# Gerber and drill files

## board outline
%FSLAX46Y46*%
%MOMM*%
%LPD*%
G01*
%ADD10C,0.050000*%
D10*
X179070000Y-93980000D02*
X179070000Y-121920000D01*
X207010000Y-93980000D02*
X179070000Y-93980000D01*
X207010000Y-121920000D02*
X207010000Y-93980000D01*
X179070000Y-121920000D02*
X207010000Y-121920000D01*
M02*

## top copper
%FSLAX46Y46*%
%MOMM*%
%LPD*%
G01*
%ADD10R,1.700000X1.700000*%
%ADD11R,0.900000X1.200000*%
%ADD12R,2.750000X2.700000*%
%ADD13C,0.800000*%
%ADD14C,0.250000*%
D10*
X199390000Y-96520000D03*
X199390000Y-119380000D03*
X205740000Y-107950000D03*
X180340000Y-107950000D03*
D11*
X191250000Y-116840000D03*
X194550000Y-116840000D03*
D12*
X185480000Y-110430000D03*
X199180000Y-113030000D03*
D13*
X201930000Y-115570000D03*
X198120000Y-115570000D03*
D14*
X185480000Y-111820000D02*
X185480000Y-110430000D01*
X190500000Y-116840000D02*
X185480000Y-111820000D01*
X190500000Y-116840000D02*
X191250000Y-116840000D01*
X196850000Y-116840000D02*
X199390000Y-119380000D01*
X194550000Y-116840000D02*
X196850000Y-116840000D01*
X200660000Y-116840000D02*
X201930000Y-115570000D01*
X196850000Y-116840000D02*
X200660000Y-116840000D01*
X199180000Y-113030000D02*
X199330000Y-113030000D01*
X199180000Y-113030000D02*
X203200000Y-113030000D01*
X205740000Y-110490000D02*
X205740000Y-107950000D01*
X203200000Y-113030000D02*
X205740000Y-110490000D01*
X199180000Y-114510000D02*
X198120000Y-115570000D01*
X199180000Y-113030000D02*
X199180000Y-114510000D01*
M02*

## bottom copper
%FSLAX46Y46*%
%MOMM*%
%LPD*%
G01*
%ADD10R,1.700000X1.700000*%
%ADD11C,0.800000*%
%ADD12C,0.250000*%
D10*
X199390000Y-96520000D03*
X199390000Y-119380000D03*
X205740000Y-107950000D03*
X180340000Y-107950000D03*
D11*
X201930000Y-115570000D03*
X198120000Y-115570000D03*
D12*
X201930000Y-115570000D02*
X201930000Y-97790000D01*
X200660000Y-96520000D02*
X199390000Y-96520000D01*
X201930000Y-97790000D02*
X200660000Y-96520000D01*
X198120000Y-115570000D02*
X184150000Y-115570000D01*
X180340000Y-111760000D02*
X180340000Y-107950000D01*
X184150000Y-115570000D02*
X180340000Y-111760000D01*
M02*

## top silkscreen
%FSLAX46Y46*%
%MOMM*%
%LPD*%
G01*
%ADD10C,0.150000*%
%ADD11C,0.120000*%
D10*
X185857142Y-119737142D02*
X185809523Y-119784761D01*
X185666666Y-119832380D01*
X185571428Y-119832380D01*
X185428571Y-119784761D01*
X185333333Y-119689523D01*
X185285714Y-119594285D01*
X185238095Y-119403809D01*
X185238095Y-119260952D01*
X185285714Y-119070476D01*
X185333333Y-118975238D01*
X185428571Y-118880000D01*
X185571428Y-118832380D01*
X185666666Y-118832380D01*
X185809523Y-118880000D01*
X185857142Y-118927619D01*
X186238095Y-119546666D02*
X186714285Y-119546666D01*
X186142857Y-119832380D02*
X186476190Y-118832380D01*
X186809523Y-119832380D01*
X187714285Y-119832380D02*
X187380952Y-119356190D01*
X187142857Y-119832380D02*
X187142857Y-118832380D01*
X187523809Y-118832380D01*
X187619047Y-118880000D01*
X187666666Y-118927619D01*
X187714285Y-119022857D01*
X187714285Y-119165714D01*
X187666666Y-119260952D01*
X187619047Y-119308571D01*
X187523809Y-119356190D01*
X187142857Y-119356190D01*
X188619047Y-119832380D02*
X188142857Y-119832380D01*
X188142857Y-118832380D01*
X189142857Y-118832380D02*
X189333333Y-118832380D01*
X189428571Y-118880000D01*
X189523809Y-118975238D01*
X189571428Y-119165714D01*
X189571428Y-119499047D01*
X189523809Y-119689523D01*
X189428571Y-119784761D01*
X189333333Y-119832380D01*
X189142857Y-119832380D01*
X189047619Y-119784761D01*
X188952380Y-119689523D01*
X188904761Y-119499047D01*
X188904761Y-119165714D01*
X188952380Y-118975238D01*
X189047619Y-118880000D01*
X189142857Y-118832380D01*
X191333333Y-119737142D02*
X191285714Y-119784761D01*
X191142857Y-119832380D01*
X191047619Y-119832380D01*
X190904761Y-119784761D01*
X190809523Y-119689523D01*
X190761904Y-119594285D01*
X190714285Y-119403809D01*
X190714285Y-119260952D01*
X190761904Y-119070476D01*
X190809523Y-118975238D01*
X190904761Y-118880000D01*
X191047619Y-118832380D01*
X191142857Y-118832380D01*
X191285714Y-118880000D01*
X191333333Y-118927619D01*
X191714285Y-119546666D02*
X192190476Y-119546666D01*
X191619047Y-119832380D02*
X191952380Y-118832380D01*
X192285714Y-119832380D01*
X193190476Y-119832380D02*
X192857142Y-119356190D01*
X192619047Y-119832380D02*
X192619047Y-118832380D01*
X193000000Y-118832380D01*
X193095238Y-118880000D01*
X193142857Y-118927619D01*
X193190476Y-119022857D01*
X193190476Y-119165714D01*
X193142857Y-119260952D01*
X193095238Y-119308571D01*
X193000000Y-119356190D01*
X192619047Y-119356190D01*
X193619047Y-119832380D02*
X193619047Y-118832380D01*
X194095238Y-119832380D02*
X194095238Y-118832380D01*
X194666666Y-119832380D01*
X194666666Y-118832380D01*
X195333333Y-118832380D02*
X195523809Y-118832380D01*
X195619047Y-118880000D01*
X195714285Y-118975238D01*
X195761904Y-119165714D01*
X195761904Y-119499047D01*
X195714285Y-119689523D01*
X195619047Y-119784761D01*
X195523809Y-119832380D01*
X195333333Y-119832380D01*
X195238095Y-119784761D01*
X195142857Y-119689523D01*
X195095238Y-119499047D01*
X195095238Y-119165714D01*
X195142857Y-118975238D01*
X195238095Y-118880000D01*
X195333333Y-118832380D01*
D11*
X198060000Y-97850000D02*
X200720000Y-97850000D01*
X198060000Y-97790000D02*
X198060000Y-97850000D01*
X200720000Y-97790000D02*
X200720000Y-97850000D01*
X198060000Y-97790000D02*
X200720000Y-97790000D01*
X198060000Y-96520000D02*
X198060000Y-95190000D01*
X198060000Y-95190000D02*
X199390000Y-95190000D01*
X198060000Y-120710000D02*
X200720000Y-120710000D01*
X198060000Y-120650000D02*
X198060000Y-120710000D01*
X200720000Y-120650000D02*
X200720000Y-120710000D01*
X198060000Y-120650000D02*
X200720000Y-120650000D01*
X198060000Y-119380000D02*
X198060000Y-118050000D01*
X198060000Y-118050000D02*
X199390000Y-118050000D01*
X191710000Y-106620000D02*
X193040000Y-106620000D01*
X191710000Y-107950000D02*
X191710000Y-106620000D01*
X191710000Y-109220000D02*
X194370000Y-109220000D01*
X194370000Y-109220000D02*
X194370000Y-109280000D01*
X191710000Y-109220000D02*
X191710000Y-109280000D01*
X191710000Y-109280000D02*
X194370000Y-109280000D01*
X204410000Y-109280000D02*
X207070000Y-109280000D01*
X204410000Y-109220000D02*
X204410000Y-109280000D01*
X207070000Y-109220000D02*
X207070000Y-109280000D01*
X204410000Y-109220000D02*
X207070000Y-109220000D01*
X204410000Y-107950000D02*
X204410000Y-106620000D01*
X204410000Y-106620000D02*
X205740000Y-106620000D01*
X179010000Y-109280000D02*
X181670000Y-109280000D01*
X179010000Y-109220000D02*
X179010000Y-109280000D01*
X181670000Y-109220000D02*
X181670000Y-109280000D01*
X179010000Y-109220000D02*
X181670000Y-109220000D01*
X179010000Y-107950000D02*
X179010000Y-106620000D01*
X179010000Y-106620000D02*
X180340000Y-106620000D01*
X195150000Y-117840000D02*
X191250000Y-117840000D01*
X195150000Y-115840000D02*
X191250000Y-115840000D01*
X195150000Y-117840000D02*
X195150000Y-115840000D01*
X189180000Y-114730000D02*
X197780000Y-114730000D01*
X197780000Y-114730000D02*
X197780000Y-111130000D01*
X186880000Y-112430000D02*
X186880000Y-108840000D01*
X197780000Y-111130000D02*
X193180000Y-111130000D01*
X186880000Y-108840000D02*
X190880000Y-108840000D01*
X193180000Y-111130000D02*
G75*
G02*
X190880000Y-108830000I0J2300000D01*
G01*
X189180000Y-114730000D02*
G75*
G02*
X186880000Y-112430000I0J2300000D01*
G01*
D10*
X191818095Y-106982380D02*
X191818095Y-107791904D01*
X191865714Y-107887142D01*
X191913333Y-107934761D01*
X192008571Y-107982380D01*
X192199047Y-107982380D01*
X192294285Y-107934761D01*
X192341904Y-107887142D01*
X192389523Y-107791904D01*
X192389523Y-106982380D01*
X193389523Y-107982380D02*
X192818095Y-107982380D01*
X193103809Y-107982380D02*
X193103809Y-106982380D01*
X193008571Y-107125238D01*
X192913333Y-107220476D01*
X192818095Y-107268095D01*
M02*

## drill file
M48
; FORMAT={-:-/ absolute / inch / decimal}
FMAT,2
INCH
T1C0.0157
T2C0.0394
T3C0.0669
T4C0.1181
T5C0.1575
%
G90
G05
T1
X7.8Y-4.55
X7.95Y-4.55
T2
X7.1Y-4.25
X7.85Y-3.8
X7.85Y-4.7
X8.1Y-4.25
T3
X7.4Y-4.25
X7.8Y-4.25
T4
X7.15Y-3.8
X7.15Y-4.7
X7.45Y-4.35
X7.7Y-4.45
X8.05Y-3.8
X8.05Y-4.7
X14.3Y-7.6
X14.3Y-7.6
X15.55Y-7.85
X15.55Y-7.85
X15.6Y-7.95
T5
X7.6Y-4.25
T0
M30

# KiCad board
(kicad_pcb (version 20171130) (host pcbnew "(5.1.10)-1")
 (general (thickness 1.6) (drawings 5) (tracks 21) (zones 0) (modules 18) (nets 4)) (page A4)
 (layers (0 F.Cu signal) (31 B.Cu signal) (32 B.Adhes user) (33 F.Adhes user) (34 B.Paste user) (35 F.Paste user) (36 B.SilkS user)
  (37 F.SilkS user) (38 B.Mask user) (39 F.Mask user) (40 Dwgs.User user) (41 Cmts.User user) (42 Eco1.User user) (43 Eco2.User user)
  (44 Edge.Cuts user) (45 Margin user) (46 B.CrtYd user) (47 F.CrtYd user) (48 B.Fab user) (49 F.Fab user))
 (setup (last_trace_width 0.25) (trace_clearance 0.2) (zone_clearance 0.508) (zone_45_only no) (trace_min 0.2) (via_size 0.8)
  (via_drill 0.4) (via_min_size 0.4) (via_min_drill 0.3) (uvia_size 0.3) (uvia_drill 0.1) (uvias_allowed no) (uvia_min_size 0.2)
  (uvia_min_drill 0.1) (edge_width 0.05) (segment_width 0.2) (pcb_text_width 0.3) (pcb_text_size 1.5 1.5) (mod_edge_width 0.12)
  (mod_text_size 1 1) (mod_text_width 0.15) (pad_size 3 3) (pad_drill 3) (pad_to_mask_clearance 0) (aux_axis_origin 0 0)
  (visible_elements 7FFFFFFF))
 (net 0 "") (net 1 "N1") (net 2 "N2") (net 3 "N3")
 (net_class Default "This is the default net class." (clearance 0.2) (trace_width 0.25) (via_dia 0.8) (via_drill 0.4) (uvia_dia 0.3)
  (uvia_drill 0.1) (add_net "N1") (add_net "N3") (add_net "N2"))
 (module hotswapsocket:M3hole (layer F.Cu) (at 204.47 96.52)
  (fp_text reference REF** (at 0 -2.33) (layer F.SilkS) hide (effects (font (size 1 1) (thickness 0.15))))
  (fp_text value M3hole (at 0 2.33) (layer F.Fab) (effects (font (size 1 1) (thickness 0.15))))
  (pad "" np_thru_hole circle (at 0 0) (size 3 3) (drill 3) (layers *.Cu *.Mask)))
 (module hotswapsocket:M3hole (layer F.Cu) (at 181.61 119.38)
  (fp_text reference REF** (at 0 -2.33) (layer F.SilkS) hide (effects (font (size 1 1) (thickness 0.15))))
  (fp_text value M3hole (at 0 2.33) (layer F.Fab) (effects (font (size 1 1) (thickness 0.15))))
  (pad "" np_thru_hole circle (at 0 0) (size 3 3) (drill 3) (layers *.Cu *.Mask)))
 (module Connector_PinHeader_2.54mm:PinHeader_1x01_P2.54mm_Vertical (layer F.Cu) (at 204.47 119.38)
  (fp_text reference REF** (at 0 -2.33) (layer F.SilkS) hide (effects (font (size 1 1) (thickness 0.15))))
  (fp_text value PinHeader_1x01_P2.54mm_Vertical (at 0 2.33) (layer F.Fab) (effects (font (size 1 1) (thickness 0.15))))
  (pad "" np_thru_hole circle (at 0 0) (size 3 3) (drill 3) (layers *.Cu *.Mask)))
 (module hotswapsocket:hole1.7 (layer F.Cu) (at 198.12 107.95)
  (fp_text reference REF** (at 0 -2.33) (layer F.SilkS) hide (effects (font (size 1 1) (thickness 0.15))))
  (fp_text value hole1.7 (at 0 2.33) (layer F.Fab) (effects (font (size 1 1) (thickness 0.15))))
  (pad "" np_thru_hole circle (at 0 0) (size 1.7 1.7) (drill 1.7) (layers *.Cu *.Mask)))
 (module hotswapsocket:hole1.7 (layer F.Cu) (at 187.96 107.95)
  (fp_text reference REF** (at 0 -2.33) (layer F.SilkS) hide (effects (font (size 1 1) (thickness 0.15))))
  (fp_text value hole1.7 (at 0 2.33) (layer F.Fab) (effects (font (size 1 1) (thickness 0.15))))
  (pad "" np_thru_hole circle (at 0 0) (size 1.7 1.7) (drill 1.7) (layers *.Cu *.Mask)))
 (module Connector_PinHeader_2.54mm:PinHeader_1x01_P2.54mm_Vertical (layer F.Cu) (at 199.39 96.52)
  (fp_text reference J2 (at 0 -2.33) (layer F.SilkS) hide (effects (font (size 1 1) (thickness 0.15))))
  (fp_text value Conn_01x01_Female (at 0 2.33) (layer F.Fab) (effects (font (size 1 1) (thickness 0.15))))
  (fp_line (start -1.33 1.33) (end 1.33 1.33) (layer F.SilkS) (width 0.12))
  (fp_line (start -1.33 1.27) (end -1.33 1.33) (layer F.SilkS) (width 0.12))
  (fp_line (start 1.33 1.27) (end 1.33 1.33) (layer F.SilkS) (width 0.12))
  (fp_line (start -1.33 1.27) (end 1.33 1.27) (layer F.SilkS) (width 0.12))
  (fp_line (start -1.33 0) (end -1.33 -1.33) (layer F.SilkS) (width 0.12))
  (fp_line (start -1.33 -1.33) (end 0 -1.33) (layer F.SilkS) (width 0.12))
  (pad 1 thru_hole rect (at 0 0) (size 1.7 1.7) (drill 1) (layers *.Cu *.Mask) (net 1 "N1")))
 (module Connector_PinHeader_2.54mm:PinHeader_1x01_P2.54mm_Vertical (layer F.Cu) (at 199.39 119.38)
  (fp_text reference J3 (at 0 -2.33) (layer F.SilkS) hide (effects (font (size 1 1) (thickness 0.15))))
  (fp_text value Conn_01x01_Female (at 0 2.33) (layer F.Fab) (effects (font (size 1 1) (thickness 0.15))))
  (fp_line (start -1.33 1.33) (end 1.33 1.33) (layer F.SilkS) (width 0.12))
  (fp_line (start -1.33 1.27) (end -1.33 1.33) (layer F.SilkS) (width 0.12))
  (fp_line (start 1.33 1.27) (end 1.33 1.33) (layer F.SilkS) (width 0.12))
  (fp_line (start -1.33 1.27) (end 1.33 1.27) (layer F.SilkS) (width 0.12))
  (fp_line (start -1.33 0) (end -1.33 -1.33) (layer F.SilkS) (width 0.12))
  (fp_line (start -1.33 -1.33) (end 0 -1.33) (layer F.SilkS) (width 0.12))
  (pad 1 thru_hole rect (at 0 0) (size 1.7 1.7) (drill 1) (layers *.Cu *.Mask) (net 1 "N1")))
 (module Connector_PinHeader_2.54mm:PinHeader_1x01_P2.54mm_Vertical (layer F.Cu) (at 193.04 107.95)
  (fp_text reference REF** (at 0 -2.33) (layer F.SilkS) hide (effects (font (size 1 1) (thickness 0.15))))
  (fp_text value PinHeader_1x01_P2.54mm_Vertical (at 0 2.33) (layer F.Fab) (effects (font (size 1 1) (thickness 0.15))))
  (fp_line (start -1.33 -1.33) (end 0 -1.33) (layer F.SilkS) (width 0.12))
  (fp_line (start -1.33 0) (end -1.33 -1.33) (layer F.SilkS) (width 0.12))
  (fp_line (start -1.33 1.27) (end 1.33 1.27) (layer F.SilkS) (width 0.12))
  (fp_line (start 1.33 1.27) (end 1.33 1.33) (layer F.SilkS) (width 0.12))
  (fp_line (start -1.33 1.27) (end -1.33 1.33) (layer F.SilkS) (width 0.12))
  (fp_line (start -1.33 1.33) (end 1.33 1.33) (layer F.SilkS) (width 0.12))
  (pad "" np_thru_hole circle (at 0 0) (size 4 4) (drill 4) (layers *.Cu *.Mask)))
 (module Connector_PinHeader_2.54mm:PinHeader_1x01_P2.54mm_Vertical (layer F.Cu) (at 205.74 107.95)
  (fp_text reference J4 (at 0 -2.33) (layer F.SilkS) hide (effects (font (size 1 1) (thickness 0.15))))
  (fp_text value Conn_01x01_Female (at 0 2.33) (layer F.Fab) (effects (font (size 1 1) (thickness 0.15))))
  (fp_line (start -1.33 1.33) (end 1.33 1.33) (layer F.SilkS) (width 0.12))
  (fp_line (start -1.33 1.27) (end -1.33 1.33) (layer F.SilkS) (width 0.12))
  (fp_line (start 1.33 1.27) (end 1.33 1.33) (layer F.SilkS) (width 0.12))
  (fp_line (start -1.33 1.27) (end 1.33 1.27) (layer F.SilkS) (width 0.12))
  (fp_line (start -1.33 0) (end -1.33 -1.33) (layer F.SilkS) (width 0.12))
  (fp_line (start -1.33 -1.33) (end 0 -1.33) (layer F.SilkS) (width 0.12))
  (pad 1 thru_hole rect (at 0 0) (size 1.7 1.7) (drill 1) (layers *.Cu *.Mask) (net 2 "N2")))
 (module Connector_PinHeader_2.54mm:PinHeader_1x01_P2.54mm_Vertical (layer F.Cu) (at 180.34 107.95)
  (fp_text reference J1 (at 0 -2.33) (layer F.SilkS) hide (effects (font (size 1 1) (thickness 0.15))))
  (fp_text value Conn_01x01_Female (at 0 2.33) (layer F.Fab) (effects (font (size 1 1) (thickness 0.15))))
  (fp_line (start -1.33 1.33) (end 1.33 1.33) (layer F.SilkS) (width 0.12))
  (fp_line (start -1.33 1.27) (end -1.33 1.33) (layer F.SilkS) (width 0.12))
  (fp_line (start 1.33 1.27) (end 1.33 1.33) (layer F.SilkS) (width 0.12))
  (fp_line (start -1.33 1.27) (end 1.33 1.27) (layer F.SilkS) (width 0.12))
  (fp_line (start -1.33 0) (end -1.33 -1.33) (layer F.SilkS) (width 0.12))
  (fp_line (start -1.33 -1.33) (end 0 -1.33) (layer F.SilkS) (width 0.12))
  (pad 1 thru_hole rect (at 0 0) (size 1.7 1.7) (drill 1) (layers *.Cu *.Mask) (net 2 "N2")))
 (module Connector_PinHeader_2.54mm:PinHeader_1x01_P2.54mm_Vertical (layer F.Cu) (at 181.61 96.52)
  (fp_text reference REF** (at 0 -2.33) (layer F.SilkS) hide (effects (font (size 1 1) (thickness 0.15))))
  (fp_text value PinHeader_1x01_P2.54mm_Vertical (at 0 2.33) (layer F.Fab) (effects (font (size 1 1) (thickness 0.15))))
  (pad "" np_thru_hole circle (at 0 0) (size 3 3) (drill 3) (layers *.Cu *.Mask)))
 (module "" (layer F.Cu) (at 214.63 105.41)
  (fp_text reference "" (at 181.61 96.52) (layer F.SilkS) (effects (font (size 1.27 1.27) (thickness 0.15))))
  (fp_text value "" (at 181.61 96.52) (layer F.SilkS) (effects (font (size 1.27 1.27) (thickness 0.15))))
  (pad "" np_thru_hole circle (at 181.61 96.52) (size 3 3) (drill 3) (layers *.Cu *.Mask)))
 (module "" (layer F.Cu) (at 213.36 102.87)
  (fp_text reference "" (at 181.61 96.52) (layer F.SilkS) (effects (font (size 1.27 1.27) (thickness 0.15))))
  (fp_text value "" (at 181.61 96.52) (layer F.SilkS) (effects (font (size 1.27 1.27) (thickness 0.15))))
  (pad "" np_thru_hole circle (at 181.61 96.52) (size 3 3) (drill 3) (layers *.Cu *.Mask)))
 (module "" (layer F.Cu) (at 213.36 102.87)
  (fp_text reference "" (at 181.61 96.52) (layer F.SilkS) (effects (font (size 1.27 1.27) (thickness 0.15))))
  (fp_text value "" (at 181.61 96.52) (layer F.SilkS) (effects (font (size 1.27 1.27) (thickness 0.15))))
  (pad "" np_thru_hole circle (at 181.61 96.52) (size 3 3) (drill 3) (layers *.Cu *.Mask)))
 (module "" (layer F.Cu) (at 181.61 96.52)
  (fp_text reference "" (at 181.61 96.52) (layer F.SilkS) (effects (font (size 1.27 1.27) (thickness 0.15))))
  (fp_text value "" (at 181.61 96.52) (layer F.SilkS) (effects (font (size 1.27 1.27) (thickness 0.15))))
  (pad "" np_thru_hole circle (at 181.61 96.52) (size 3 3) (drill 3) (layers *.Cu *.Mask)))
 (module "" (layer F.Cu) (at 181.61 96.52)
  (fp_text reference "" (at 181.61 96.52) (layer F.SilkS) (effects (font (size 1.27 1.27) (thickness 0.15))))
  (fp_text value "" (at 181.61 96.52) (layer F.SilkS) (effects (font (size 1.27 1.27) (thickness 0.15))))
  (pad "" np_thru_hole circle (at 181.61 96.52) (size 3 3) (drill 3) (layers *.Cu *.Mask)))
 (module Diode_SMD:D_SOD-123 (layer F.Cu) (at 192.9 116.84 180)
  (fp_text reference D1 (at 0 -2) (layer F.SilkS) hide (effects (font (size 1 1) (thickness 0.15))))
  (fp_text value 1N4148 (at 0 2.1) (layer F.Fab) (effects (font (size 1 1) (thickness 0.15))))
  (fp_line (start -2.25 -1) (end 1.65 -1) (layer F.SilkS) (width 0.12))
  (fp_line (start -2.25 1) (end 1.65 1) (layer F.SilkS) (width 0.12))
  (fp_line (start -2.25 -1) (end -2.25 1) (layer F.SilkS) (width 0.12))
  (pad 2 smd rect (at 1.65 0 180) (size 0.9 1.2) (layers F.Cu F.Paste F.Mask) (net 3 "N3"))
  (pad 1 smd rect (at -1.65 0 180) (size 0.9 1.2) (layers F.Cu F.Paste F.Mask) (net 1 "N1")))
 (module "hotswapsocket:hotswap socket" (layer F.Cu) (at 192.58 112.53)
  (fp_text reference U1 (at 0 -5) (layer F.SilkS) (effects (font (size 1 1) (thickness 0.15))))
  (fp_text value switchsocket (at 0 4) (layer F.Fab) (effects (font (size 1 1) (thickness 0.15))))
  (fp_line (start -3.4 2.2) (end 5.2 2.2) (layer F.SilkS) (width 0.12))
  (fp_line (start 5.2 2.2) (end 5.2 -1.4) (layer F.SilkS) (width 0.12))
  (fp_line (start -5.7 -0.1) (end -5.7 -3.69) (layer F.SilkS) (width 0.12))
  (fp_line (start 5.2 -1.4) (end 0.6 -1.4) (layer F.SilkS) (width 0.12))
  (fp_line (start -5.7 -3.69) (end -1.7 -3.69) (layer F.SilkS) (width 0.12))
  (fp_arc (start 0.6 -3.7) (end -1.7 -3.7) (angle -90) (layer F.SilkS) (width 0.12))
  (fp_arc (start -3.4 -0.1) (end -5.7 -0.1) (angle -90) (layer F.SilkS) (width 0.12))
  (pad 2 smd rect (at -7.1 -2.1) (size 2.75 2.7) (layers F.Cu F.Paste F.Mask) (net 3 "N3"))
  (pad 1 smd rect (at 6.6 0.5) (size 2.75 2.7) (layers F.Cu F.Paste F.Mask) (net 2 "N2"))
  (pad "" np_thru_hole circle (at -3.35 -2.04) (size 3 3) (drill 3) (layers *.Cu *.Mask))
  (pad "" np_thru_hole circle (at 3 0.5) (size 3 3) (drill 3) (layers *.Cu *.Mask)))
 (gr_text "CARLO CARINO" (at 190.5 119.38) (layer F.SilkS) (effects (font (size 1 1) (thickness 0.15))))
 (gr_line (start 179.07 93.98) (end 179.07 121.92) (layer Edge.Cuts) (width 0.05))
 (gr_line (start 207.01 93.98) (end 179.07 93.98) (layer Edge.Cuts) (width 0.05))
 (gr_line (start 207.01 121.92) (end 207.01 93.98) (layer Edge.Cuts) (width 0.05))
 (gr_line (start 179.07 121.92) (end 207.01 121.92) (layer Edge.Cuts) (width 0.05))
 (segment (start 185.48 111.82) (end 185.48 110.43) (width 0.25) (layer F.Cu) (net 3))
 (segment (start 190.5 116.84) (end 185.48 111.82) (width 0.25) (layer F.Cu) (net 3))
 (segment (start 190.5 116.84) (end 191.25 116.84) (width 0.25) (layer F.Cu) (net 3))
 (segment (start 196.85 116.84) (end 199.39 119.38) (width 0.25) (layer F.Cu) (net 1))
 (segment (start 194.55 116.84) (end 196.85 116.84) (width 0.25) (layer F.Cu) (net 1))
 (via (at 201.93 115.57) (size 0.8) (drill 0.4) (layers F.Cu B.Cu) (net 1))
 (segment (start 200.66 116.84) (end 201.93 115.57) (width 0.25) (layer F.Cu) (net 1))
 (segment (start 196.85 116.84) (end 200.66 116.84) (width 0.25) (layer F.Cu) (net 1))
 (segment (start 201.93 115.57) (end 201.93 97.79) (width 0.25) (layer B.Cu) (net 1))
 (segment (start 200.66 96.52) (end 199.39 96.52) (width 0.25) (layer B.Cu) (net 1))
 (segment (start 201.93 97.79) (end 200.66 96.52) (width 0.25) (layer B.Cu) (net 1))
 (segment (start 199.18 113.03) (end 199.33 113.03) (width 0.25) (layer F.Cu) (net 2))
 (segment (start 199.18 113.03) (end 203.2 113.03) (width 0.25) (layer F.Cu) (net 2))
 (segment (start 205.74 110.49) (end 205.74 107.95) (width 0.25) (layer F.Cu) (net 2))
 (segment (start 203.2 113.03) (end 205.74 110.49) (width 0.25) (layer F.Cu) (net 2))
 (via (at 198.12 115.57) (size 0.8) (drill 0.4) (layers F.Cu B.Cu) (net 2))
 (segment (start 199.18 114.51) (end 198.12 115.57) (width 0.25) (layer F.Cu) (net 2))
 (segment (start 199.18 113.03) (end 199.18 114.51) (width 0.25) (layer F.Cu) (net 2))
 (segment (start 198.12 115.57) (end 184.15 115.57) (width 0.25) (layer B.Cu) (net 2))
 (segment (start 180.34 111.76) (end 180.34 107.95) (width 0.25) (layer B.Cu) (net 2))
 (segment (start 184.15 115.57) (end 180.34 111.76) (width 0.25) (layer B.Cu) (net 2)))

